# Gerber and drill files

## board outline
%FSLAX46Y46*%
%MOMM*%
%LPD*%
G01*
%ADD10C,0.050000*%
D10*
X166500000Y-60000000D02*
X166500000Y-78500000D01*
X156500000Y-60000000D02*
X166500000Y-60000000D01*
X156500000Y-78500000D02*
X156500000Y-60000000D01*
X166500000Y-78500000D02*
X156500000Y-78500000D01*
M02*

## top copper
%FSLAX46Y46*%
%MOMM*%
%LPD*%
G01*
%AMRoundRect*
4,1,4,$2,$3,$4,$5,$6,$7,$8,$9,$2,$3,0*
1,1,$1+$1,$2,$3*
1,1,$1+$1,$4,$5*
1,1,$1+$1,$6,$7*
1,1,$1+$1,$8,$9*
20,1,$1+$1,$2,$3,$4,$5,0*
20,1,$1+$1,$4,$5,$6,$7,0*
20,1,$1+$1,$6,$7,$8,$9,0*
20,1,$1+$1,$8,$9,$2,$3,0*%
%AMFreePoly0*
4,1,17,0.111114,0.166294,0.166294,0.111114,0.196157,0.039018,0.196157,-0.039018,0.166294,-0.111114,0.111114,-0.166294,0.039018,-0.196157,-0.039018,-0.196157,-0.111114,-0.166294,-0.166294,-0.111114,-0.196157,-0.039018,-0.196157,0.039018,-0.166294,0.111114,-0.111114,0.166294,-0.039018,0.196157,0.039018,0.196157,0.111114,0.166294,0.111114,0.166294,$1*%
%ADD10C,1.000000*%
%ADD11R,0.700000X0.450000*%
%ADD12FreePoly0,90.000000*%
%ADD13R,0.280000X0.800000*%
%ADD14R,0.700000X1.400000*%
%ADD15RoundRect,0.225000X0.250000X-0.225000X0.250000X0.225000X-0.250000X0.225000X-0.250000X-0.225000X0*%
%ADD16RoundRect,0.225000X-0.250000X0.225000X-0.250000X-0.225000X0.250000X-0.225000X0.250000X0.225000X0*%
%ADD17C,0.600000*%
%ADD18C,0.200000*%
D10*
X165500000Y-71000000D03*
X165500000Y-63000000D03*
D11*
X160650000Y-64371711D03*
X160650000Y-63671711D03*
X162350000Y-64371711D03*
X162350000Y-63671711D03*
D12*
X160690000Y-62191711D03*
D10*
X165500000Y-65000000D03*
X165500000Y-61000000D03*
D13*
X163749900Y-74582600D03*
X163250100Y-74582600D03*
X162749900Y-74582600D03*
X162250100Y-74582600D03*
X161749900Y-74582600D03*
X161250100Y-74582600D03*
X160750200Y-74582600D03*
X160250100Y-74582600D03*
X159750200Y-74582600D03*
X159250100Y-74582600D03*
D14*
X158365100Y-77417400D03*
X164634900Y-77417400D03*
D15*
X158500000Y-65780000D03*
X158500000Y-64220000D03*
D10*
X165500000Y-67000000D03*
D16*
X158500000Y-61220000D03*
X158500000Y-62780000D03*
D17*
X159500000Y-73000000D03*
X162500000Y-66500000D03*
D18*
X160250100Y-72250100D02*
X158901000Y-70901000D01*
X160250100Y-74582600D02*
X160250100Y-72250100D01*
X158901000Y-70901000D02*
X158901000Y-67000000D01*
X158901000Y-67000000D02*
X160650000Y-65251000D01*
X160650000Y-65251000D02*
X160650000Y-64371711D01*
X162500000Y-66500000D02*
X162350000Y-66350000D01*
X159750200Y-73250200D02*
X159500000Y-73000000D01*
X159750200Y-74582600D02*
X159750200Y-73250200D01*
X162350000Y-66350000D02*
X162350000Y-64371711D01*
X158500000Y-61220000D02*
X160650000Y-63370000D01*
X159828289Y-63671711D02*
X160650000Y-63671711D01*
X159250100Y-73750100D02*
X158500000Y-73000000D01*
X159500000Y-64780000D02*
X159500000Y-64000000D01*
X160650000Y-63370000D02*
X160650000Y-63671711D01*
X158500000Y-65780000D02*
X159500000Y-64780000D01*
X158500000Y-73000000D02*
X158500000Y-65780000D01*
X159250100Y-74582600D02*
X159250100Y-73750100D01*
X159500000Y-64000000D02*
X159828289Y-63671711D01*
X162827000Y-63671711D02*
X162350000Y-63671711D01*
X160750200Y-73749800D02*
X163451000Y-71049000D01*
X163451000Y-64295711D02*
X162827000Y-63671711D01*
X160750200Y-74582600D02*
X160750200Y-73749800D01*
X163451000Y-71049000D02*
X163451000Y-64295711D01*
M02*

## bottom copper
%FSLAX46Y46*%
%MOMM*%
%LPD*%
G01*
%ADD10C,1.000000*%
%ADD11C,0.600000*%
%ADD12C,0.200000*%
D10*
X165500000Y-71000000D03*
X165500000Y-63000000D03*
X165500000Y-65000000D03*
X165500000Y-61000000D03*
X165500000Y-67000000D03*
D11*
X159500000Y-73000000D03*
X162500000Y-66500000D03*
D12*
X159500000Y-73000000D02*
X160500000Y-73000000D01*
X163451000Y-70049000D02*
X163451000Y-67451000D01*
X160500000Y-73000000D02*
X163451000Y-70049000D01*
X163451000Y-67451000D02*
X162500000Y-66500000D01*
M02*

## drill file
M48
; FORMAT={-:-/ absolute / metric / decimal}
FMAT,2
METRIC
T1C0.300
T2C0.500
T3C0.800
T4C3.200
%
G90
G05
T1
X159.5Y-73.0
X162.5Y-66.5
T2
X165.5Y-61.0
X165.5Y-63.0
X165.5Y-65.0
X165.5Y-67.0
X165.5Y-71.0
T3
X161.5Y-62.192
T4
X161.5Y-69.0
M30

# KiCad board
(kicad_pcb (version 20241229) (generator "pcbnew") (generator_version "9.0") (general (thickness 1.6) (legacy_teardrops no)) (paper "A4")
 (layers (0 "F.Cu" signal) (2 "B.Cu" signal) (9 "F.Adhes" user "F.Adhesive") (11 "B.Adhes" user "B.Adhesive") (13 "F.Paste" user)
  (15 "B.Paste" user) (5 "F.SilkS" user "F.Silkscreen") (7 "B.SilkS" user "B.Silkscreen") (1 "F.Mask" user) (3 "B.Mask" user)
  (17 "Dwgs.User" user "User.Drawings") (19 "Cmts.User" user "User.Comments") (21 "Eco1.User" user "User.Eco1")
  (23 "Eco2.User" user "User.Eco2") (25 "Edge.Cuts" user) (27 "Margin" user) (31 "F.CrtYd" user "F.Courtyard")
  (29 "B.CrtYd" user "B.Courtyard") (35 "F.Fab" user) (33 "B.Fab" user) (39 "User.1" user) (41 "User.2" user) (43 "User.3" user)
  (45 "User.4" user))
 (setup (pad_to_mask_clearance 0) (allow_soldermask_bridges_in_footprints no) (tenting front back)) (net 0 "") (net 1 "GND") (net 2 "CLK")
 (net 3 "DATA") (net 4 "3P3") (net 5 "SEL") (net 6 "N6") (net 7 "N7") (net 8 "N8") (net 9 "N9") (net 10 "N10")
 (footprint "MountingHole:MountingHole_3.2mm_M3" (layer "F.Cu") (at 161.5 69)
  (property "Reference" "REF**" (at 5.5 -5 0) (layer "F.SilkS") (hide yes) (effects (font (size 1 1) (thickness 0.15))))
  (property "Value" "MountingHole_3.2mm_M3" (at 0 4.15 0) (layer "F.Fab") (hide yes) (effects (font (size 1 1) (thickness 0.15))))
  (pad "" np_thru_hole circle (at 0 0) (size 3.2 3.2) (drill 3.2) (layers "*.Cu" "*.Mask")))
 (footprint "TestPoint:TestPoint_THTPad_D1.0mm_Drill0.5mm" (layer "F.Cu") (at 165.5 71)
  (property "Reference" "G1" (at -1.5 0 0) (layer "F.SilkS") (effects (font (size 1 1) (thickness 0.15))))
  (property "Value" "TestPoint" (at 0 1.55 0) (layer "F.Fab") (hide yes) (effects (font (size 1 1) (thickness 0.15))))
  (pad "1" thru_hole circle (at 0 0) (size 1 1) (drill 0.5) (layers "*.Cu" "*.Mask") (remove_unused_layers no) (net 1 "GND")))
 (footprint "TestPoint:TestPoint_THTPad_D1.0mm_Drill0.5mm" (layer "F.Cu") (at 165.5 63)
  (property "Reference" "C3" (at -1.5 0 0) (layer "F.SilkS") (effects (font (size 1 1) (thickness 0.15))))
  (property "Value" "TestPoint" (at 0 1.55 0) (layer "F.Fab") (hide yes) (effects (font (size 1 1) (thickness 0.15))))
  (pad "1" thru_hole circle (at 0 0) (size 1 1) (drill 0.5) (layers "*.Cu" "*.Mask") (remove_unused_layers no) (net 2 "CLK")))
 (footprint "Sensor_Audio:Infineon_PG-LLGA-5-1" (layer "F.Cu") (at 161.5 62.871711 90)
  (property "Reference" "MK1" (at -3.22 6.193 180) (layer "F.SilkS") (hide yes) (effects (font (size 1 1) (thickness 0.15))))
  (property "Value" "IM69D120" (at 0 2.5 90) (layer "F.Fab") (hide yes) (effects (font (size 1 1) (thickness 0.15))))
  (pad "" smd custom (at -1.5 -0.725 90) (size 0.3 0.3) (layers "F.Paste") (zone_connect 0) (options (clearance outline) (anchor circle))
   (primitives))
  (pad "" smd custom (at -1.5 0.725 90) (size 0.3 0.3) (layers "F.Paste") (zone_connect 0) (options (clearance outline) (anchor circle))
   (primitives))
  (pad "" smd custom (at -0.8 -0.725 90) (size 0.3 0.3) (layers "F.Paste") (zone_connect 0) (options (clearance outline) (anchor circle))
   (primitives))
  (pad "" smd custom (at -0.8 0.725 90) (size 0.3 0.3) (layers "F.Paste") (zone_connect 0) (options (clearance outline) (anchor circle))
   (primitives))
  (pad "" smd custom (at -0.12 0 90) (size 0.3 0.3) (layers "F.Paste") (zone_connect 0) (options (clearance outline) (anchor circle))
   (primitives))
  (pad "" smd custom (at 0.28 -0.693 90) (size 0.3 0.3) (layers "F.Paste") (zone_connect 0) (options (clearance outline) (anchor circle))
   (primitives))
  (pad "" smd custom (at 0.28 0.693 90) (size 0.3 0.3) (layers "F.Paste") (zone_connect 0) (options (clearance outline) (anchor circle))
   (primitives))
  (pad "" np_thru_hole circle (at 0.68 0 90) (size 0.8 0.8) (drill 0.8) (layers "*.Cu" "*.Mask"))
  (pad "" smd custom (at 1.08 -0.693 90) (size 0.3 0.3) (layers "F.Paste") (zone_connect 0) (options (clearance outline) (anchor circle))
   (primitives))
  (pad "" smd custom (at 1.08 0.693 90) (size 0.3 0.3) (layers "F.Paste") (zone_connect 0) (options (clearance outline) (anchor circle))
   (primitives))
  (pad "" smd custom (at 1.48 0 90) (size 0.3 0.3) (layers "F.Paste") (zone_connect 0) (options (clearance outline) (anchor circle))
   (primitives))
  (pad "1" smd rect (at -1.5 -0.85 90) (size 0.45 0.7) (layers "F.Cu" "F.Mask") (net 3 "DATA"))
  (pad "2" smd rect (at -0.8 -0.85 90) (size 0.45 0.7) (layers "F.Cu" "F.Mask") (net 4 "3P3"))
  (pad "3" smd rect (at -1.5 0.85 90) (size 0.45 0.7) (layers "F.Cu" "F.Mask") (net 2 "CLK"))
  (pad "4" smd rect (at -0.8 0.85 90) (size 0.45 0.7) (layers "F.Cu" "F.Mask") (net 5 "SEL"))
  (pad "5" smd custom (at 0.68 -0.81 90) (size 0.4 0.4) (layers "F.Cu" "F.Mask") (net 1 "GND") (zone_connect 0)
   (options (clearance outline) (anchor circle)) (primitives)))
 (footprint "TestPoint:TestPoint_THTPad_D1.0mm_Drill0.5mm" (layer "F.Cu") (at 165.5 65)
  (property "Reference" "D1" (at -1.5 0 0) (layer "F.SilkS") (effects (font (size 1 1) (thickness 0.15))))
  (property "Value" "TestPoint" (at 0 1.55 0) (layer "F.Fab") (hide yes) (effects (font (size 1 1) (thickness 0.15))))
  (pad "1" thru_hole circle (at 0 0) (size 1 1) (drill 0.5) (layers "*.Cu" "*.Mask") (remove_unused_layers no) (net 3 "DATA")))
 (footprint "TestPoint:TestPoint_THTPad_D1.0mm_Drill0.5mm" (layer "F.Cu") (at 165.5 61)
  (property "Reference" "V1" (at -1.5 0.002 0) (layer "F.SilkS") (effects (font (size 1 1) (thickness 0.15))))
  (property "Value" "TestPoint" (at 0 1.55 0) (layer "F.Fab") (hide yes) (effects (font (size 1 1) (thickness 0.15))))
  (pad "1" thru_hole circle (at 0 0) (size 1 1) (drill 0.5) (layers "*.Cu" "*.Mask") (remove_unused_layers no) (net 4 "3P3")))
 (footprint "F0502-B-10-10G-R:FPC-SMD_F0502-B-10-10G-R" (layer "F.Cu") (at 161.5 76)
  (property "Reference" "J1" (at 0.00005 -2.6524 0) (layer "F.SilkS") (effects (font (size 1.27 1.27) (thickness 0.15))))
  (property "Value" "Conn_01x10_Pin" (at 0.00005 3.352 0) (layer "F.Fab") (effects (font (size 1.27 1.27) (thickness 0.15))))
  (pad "1" smd rect (at 2.2499 -1.4174) (size 0.28 0.8) (layers "F.Cu" "F.Mask" "F.Paste") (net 1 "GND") (solder_mask_margin 0.0508)
   (solder_paste_margin 0) (thermal_bridge_angle 0))
  (pad "2" smd rect (at 1.7501 -1.4174) (size 0.28 0.8) (layers "F.Cu" "F.Mask" "F.Paste") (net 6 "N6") (solder_mask_margin 0.0508)
   (solder_paste_margin 0) (thermal_bridge_angle 0))
  (pad "3" smd rect (at 1.2499 -1.4174) (size 0.28 0.8) (layers "F.Cu" "F.Mask" "F.Paste") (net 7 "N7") (solder_mask_margin 0.0508)
   (solder_paste_margin 0) (thermal_bridge_angle 0))
  (pad "4" smd rect (at 0.7501 -1.4174) (size 0.28 0.8) (layers "F.Cu" "F.Mask" "F.Paste") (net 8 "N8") (solder_mask_margin 0.0508)
   (solder_paste_margin 0) (thermal_bridge_angle 0))
  (pad "5" smd rect (at 0.2499 -1.4174) (size 0.28 0.8) (layers "F.Cu" "F.Mask" "F.Paste") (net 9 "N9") (solder_mask_margin 0.0508)
   (solder_paste_margin 0) (thermal_bridge_angle 0))
  (pad "6" smd rect (at -0.2499 -1.4174) (size 0.28 0.8) (layers "F.Cu" "F.Mask" "F.Paste") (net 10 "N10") (solder_mask_margin 0.0508)
   (solder_paste_margin 0) (thermal_bridge_angle 0))
  (pad "7" smd rect (at -0.7498 -1.4174) (size 0.28 0.8) (layers "F.Cu" "F.Mask" "F.Paste") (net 5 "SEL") (solder_mask_margin 0.0508)
   (solder_paste_margin 0) (thermal_bridge_angle 0))
  (pad "8" smd rect (at -1.2499 -1.4174) (size 0.28 0.8) (layers "F.Cu" "F.Mask" "F.Paste") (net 3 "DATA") (solder_mask_margin 0.0508)
   (solder_paste_margin 0) (thermal_bridge_angle 0))
  (pad "9" smd rect (at -1.7498 -1.4174) (size 0.28 0.8) (layers "F.Cu" "F.Mask" "F.Paste") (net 2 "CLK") (solder_mask_margin 0.0508)
   (solder_paste_margin 0) (thermal_bridge_angle 0))
  (pad "10" smd rect (at -2.2499 -1.4174) (size 0.28 0.8) (layers "F.Cu" "F.Mask" "F.Paste") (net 4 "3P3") (solder_mask_margin 0.0508)
   (solder_paste_margin 0) (thermal_bridge_angle 0))
  (pad "11" smd rect (at -3.1349 1.4174) (size 0.7 1.4) (layers "F.Cu" "F.Mask" "F.Paste") (solder_mask_margin 0.0508)
   (solder_paste_margin 0) (thermal_bridge_angle 0))
  (pad "12" smd rect (at 3.1349 1.4174) (size 0.7 1.4) (layers "F.Cu" "F.Mask" "F.Paste") (solder_mask_margin 0.0508)
   (solder_paste_margin 0) (thermal_bridge_angle 0))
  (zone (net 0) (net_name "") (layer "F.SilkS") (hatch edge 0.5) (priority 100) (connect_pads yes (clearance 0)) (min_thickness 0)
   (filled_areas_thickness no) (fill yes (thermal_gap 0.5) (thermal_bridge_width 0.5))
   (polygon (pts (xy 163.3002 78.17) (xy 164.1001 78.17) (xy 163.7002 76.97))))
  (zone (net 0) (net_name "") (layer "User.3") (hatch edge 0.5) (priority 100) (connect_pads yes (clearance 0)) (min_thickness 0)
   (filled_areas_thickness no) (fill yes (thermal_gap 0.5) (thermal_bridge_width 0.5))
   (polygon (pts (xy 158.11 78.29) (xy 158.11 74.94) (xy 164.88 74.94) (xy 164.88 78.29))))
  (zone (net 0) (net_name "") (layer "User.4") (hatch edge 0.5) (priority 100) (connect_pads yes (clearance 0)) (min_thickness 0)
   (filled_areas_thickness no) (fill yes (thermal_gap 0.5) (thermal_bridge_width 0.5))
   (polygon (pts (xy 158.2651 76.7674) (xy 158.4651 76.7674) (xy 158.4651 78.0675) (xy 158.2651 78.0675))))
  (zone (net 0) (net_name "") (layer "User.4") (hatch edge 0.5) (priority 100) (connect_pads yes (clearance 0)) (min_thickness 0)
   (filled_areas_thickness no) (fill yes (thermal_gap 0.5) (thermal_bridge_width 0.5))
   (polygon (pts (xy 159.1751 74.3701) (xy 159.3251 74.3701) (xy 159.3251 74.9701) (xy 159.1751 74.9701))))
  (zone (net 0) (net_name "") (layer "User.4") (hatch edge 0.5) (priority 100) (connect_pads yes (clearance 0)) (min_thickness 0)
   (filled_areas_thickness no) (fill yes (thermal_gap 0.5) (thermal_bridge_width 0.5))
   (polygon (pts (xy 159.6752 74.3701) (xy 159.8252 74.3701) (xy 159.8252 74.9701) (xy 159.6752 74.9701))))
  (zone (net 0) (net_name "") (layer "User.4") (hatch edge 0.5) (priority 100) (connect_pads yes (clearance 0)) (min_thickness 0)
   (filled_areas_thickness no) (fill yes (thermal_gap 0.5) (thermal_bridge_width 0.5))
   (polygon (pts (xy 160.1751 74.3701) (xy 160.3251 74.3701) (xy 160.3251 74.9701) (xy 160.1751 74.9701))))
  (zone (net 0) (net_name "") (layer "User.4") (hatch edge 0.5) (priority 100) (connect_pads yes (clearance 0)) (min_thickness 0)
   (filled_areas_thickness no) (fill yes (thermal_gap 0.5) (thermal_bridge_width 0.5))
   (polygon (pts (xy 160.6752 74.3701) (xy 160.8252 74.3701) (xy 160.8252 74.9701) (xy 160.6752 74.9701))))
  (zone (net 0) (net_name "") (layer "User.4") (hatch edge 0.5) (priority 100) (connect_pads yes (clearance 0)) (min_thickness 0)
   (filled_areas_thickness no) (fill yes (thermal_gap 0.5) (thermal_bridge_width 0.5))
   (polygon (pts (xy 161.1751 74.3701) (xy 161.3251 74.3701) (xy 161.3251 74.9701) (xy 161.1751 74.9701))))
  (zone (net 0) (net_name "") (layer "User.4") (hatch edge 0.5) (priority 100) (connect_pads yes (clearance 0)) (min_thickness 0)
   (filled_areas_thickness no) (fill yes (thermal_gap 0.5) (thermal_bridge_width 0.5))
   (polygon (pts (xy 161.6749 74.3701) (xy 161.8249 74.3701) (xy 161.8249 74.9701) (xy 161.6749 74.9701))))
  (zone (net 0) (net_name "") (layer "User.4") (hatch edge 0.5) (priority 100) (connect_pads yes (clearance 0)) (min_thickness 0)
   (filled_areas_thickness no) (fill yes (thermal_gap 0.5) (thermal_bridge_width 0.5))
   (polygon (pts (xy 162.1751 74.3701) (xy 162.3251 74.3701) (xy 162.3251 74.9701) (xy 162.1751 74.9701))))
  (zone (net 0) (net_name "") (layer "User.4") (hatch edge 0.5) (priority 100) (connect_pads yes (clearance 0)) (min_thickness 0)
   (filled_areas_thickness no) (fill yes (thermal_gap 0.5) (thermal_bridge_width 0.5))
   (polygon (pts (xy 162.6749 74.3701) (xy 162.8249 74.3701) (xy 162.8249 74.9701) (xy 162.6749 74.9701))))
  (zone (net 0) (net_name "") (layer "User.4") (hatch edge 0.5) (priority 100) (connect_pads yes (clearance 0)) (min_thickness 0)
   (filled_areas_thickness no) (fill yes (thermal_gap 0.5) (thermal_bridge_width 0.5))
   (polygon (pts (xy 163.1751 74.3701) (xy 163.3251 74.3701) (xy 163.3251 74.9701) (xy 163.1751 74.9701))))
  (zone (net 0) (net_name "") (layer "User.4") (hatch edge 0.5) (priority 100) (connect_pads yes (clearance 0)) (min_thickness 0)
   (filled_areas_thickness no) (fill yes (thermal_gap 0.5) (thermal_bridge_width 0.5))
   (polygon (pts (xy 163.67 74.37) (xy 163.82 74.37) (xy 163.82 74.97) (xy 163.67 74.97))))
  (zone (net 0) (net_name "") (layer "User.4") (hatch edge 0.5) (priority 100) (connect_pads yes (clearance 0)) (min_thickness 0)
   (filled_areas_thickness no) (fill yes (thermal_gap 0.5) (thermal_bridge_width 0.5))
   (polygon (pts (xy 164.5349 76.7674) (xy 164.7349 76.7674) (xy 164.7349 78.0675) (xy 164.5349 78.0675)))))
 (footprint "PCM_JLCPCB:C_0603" (layer "F.Cu") (at 158.5 65 90)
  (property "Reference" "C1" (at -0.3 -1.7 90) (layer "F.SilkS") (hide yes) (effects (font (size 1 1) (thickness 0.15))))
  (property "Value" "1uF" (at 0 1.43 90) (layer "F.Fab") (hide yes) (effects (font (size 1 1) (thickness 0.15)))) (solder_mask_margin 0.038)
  (pad "1" smd roundrect (at -0.78 0 90) (size 0.9 0.95) (layers "F.Cu" "F.Mask" "F.Paste") (roundrect_rratio 0.25) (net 4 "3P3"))
  (pad "2" smd roundrect (at 0.78 0 90) (size 0.9 0.95) (layers "F.Cu" "F.Mask" "F.Paste") (roundrect_rratio 0.25) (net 1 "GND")))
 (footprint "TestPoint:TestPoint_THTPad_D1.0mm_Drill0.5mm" (layer "F.Cu") (at 165.5 67)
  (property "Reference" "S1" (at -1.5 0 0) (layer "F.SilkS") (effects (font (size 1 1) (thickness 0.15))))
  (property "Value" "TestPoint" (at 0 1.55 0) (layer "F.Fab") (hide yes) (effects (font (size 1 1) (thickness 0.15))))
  (pad "1" thru_hole circle (at 0 0) (size 1 1) (drill 0.5) (layers "*.Cu" "*.Mask") (remove_unused_layers no) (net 5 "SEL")))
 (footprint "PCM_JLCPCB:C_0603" (layer "F.Cu") (at 158.5 62 -90)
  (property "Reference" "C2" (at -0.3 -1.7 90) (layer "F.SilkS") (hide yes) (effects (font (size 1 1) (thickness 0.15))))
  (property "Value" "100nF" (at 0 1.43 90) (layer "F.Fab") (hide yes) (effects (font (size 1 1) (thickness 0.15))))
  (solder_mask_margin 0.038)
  (pad "1" smd roundrect (at -0.78 0 270) (size 0.9 0.95) (layers "F.Cu" "F.Mask" "F.Paste") (roundrect_rratio 0.25) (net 4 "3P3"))
  (pad "2" smd roundrect (at 0.78 0 270) (size 0.9 0.95) (layers "F.Cu" "F.Mask" "F.Paste") (roundrect_rratio 0.25) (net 1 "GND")))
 (gr_line (start 166.5 60) (end 166.5 78.5) (stroke (width 0.05) (type default)) (layer "Edge.Cuts"))
 (gr_line (start 156.5 60) (end 166.5 60) (stroke (width 0.05) (type default)) (layer "Edge.Cuts"))
 (gr_line (start 156.5 78.5) (end 156.5 60) (stroke (width 0.05) (type default)) (layer "Edge.Cuts"))
 (gr_line (start 166.5 78.5) (end 156.5 78.5) (stroke (width 0.05) (type default)) (layer "Edge.Cuts"))
 (segment (start 160.2501 72.2501) (end 158.901 70.901) (width 0.2) (layer "F.Cu") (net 3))
 (segment (start 160.2501 74.5826) (end 160.2501 72.2501) (width 0.2) (layer "F.Cu") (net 3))
 (segment (start 158.901 70.901) (end 158.901 67) (width 0.2) (layer "F.Cu") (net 3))
 (segment (start 158.901 67) (end 160.65 65.251) (width 0.2) (layer "F.Cu") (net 3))
 (segment (start 160.65 65.251) (end 160.65 64.371711) (width 0.2) (layer "F.Cu") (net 3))
 (segment (start 162.5 66.5) (end 162.35 66.35) (width 0.2) (layer "F.Cu") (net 2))
 (segment (start 159.7502 73.2502) (end 159.5 73) (width 0.2) (layer "F.Cu") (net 2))
 (segment (start 159.7502 74.5826) (end 159.7502 73.2502) (width 0.2) (layer "F.Cu") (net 2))
 (segment (start 162.35 66.35) (end 162.35 64.371711) (width 0.2) (layer "F.Cu") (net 2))
 (via (at 159.5 73) (size 0.6) (drill 0.3) (layers "F.Cu" "B.Cu") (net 2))
 (via (at 162.5 66.5) (size 0.6) (drill 0.3) (layers "F.Cu" "B.Cu") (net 2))
 (segment (start 159.5 73) (end 160.5 73) (width 0.2) (layer "B.Cu") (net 2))
 (segment (start 163.451 70.049) (end 163.451 67.451) (width 0.2) (layer "B.Cu") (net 2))
 (segment (start 160.5 73) (end 163.451 70.049) (width 0.2) (layer "B.Cu") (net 2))
 (segment (start 163.451 67.451) (end 162.5 66.5) (width 0.2) (layer "B.Cu") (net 2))
 (segment (start 158.5 61.22) (end 160.65 63.37) (width 0.2) (layer "F.Cu") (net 4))
 (segment (start 159.828289 63.671711) (end 160.65 63.671711) (width 0.2) (layer "F.Cu") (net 4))
 (segment (start 159.2501 73.7501) (end 158.5 73) (width 0.2) (layer "F.Cu") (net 4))
 (segment (start 159.5 64.78) (end 159.5 64) (width 0.2) (layer "F.Cu") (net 4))
 (segment (start 160.65 63.37) (end 160.65 63.671711) (width 0.2) (layer "F.Cu") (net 4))
 (segment (start 158.5 65.78) (end 159.5 64.78) (width 0.2) (layer "F.Cu") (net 4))
 (segment (start 158.5 73) (end 158.5 65.78) (width 0.2) (layer "F.Cu") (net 4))
 (segment (start 159.2501 74.5826) (end 159.2501 73.7501) (width 0.2) (layer "F.Cu") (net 4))
 (segment (start 159.5 64) (end 159.828289 63.671711) (width 0.2) (layer "F.Cu") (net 4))
 (segment (start 162.827 63.671711) (end 162.35 63.671711) (width 0.2) (layer "F.Cu") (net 5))
 (segment (start 160.7502 73.7498) (end 163.451 71.049) (width 0.2) (layer "F.Cu") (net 5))
 (segment (start 163.451 64.295711) (end 162.827 63.671711) (width 0.2) (layer "F.Cu") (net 5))
 (segment (start 160.7502 74.5826) (end 160.7502 73.7498) (width 0.2) (layer "F.Cu") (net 5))
 (segment (start 163.451 71.049) (end 163.451 64.295711) (width 0.2) (layer "F.Cu") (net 5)))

